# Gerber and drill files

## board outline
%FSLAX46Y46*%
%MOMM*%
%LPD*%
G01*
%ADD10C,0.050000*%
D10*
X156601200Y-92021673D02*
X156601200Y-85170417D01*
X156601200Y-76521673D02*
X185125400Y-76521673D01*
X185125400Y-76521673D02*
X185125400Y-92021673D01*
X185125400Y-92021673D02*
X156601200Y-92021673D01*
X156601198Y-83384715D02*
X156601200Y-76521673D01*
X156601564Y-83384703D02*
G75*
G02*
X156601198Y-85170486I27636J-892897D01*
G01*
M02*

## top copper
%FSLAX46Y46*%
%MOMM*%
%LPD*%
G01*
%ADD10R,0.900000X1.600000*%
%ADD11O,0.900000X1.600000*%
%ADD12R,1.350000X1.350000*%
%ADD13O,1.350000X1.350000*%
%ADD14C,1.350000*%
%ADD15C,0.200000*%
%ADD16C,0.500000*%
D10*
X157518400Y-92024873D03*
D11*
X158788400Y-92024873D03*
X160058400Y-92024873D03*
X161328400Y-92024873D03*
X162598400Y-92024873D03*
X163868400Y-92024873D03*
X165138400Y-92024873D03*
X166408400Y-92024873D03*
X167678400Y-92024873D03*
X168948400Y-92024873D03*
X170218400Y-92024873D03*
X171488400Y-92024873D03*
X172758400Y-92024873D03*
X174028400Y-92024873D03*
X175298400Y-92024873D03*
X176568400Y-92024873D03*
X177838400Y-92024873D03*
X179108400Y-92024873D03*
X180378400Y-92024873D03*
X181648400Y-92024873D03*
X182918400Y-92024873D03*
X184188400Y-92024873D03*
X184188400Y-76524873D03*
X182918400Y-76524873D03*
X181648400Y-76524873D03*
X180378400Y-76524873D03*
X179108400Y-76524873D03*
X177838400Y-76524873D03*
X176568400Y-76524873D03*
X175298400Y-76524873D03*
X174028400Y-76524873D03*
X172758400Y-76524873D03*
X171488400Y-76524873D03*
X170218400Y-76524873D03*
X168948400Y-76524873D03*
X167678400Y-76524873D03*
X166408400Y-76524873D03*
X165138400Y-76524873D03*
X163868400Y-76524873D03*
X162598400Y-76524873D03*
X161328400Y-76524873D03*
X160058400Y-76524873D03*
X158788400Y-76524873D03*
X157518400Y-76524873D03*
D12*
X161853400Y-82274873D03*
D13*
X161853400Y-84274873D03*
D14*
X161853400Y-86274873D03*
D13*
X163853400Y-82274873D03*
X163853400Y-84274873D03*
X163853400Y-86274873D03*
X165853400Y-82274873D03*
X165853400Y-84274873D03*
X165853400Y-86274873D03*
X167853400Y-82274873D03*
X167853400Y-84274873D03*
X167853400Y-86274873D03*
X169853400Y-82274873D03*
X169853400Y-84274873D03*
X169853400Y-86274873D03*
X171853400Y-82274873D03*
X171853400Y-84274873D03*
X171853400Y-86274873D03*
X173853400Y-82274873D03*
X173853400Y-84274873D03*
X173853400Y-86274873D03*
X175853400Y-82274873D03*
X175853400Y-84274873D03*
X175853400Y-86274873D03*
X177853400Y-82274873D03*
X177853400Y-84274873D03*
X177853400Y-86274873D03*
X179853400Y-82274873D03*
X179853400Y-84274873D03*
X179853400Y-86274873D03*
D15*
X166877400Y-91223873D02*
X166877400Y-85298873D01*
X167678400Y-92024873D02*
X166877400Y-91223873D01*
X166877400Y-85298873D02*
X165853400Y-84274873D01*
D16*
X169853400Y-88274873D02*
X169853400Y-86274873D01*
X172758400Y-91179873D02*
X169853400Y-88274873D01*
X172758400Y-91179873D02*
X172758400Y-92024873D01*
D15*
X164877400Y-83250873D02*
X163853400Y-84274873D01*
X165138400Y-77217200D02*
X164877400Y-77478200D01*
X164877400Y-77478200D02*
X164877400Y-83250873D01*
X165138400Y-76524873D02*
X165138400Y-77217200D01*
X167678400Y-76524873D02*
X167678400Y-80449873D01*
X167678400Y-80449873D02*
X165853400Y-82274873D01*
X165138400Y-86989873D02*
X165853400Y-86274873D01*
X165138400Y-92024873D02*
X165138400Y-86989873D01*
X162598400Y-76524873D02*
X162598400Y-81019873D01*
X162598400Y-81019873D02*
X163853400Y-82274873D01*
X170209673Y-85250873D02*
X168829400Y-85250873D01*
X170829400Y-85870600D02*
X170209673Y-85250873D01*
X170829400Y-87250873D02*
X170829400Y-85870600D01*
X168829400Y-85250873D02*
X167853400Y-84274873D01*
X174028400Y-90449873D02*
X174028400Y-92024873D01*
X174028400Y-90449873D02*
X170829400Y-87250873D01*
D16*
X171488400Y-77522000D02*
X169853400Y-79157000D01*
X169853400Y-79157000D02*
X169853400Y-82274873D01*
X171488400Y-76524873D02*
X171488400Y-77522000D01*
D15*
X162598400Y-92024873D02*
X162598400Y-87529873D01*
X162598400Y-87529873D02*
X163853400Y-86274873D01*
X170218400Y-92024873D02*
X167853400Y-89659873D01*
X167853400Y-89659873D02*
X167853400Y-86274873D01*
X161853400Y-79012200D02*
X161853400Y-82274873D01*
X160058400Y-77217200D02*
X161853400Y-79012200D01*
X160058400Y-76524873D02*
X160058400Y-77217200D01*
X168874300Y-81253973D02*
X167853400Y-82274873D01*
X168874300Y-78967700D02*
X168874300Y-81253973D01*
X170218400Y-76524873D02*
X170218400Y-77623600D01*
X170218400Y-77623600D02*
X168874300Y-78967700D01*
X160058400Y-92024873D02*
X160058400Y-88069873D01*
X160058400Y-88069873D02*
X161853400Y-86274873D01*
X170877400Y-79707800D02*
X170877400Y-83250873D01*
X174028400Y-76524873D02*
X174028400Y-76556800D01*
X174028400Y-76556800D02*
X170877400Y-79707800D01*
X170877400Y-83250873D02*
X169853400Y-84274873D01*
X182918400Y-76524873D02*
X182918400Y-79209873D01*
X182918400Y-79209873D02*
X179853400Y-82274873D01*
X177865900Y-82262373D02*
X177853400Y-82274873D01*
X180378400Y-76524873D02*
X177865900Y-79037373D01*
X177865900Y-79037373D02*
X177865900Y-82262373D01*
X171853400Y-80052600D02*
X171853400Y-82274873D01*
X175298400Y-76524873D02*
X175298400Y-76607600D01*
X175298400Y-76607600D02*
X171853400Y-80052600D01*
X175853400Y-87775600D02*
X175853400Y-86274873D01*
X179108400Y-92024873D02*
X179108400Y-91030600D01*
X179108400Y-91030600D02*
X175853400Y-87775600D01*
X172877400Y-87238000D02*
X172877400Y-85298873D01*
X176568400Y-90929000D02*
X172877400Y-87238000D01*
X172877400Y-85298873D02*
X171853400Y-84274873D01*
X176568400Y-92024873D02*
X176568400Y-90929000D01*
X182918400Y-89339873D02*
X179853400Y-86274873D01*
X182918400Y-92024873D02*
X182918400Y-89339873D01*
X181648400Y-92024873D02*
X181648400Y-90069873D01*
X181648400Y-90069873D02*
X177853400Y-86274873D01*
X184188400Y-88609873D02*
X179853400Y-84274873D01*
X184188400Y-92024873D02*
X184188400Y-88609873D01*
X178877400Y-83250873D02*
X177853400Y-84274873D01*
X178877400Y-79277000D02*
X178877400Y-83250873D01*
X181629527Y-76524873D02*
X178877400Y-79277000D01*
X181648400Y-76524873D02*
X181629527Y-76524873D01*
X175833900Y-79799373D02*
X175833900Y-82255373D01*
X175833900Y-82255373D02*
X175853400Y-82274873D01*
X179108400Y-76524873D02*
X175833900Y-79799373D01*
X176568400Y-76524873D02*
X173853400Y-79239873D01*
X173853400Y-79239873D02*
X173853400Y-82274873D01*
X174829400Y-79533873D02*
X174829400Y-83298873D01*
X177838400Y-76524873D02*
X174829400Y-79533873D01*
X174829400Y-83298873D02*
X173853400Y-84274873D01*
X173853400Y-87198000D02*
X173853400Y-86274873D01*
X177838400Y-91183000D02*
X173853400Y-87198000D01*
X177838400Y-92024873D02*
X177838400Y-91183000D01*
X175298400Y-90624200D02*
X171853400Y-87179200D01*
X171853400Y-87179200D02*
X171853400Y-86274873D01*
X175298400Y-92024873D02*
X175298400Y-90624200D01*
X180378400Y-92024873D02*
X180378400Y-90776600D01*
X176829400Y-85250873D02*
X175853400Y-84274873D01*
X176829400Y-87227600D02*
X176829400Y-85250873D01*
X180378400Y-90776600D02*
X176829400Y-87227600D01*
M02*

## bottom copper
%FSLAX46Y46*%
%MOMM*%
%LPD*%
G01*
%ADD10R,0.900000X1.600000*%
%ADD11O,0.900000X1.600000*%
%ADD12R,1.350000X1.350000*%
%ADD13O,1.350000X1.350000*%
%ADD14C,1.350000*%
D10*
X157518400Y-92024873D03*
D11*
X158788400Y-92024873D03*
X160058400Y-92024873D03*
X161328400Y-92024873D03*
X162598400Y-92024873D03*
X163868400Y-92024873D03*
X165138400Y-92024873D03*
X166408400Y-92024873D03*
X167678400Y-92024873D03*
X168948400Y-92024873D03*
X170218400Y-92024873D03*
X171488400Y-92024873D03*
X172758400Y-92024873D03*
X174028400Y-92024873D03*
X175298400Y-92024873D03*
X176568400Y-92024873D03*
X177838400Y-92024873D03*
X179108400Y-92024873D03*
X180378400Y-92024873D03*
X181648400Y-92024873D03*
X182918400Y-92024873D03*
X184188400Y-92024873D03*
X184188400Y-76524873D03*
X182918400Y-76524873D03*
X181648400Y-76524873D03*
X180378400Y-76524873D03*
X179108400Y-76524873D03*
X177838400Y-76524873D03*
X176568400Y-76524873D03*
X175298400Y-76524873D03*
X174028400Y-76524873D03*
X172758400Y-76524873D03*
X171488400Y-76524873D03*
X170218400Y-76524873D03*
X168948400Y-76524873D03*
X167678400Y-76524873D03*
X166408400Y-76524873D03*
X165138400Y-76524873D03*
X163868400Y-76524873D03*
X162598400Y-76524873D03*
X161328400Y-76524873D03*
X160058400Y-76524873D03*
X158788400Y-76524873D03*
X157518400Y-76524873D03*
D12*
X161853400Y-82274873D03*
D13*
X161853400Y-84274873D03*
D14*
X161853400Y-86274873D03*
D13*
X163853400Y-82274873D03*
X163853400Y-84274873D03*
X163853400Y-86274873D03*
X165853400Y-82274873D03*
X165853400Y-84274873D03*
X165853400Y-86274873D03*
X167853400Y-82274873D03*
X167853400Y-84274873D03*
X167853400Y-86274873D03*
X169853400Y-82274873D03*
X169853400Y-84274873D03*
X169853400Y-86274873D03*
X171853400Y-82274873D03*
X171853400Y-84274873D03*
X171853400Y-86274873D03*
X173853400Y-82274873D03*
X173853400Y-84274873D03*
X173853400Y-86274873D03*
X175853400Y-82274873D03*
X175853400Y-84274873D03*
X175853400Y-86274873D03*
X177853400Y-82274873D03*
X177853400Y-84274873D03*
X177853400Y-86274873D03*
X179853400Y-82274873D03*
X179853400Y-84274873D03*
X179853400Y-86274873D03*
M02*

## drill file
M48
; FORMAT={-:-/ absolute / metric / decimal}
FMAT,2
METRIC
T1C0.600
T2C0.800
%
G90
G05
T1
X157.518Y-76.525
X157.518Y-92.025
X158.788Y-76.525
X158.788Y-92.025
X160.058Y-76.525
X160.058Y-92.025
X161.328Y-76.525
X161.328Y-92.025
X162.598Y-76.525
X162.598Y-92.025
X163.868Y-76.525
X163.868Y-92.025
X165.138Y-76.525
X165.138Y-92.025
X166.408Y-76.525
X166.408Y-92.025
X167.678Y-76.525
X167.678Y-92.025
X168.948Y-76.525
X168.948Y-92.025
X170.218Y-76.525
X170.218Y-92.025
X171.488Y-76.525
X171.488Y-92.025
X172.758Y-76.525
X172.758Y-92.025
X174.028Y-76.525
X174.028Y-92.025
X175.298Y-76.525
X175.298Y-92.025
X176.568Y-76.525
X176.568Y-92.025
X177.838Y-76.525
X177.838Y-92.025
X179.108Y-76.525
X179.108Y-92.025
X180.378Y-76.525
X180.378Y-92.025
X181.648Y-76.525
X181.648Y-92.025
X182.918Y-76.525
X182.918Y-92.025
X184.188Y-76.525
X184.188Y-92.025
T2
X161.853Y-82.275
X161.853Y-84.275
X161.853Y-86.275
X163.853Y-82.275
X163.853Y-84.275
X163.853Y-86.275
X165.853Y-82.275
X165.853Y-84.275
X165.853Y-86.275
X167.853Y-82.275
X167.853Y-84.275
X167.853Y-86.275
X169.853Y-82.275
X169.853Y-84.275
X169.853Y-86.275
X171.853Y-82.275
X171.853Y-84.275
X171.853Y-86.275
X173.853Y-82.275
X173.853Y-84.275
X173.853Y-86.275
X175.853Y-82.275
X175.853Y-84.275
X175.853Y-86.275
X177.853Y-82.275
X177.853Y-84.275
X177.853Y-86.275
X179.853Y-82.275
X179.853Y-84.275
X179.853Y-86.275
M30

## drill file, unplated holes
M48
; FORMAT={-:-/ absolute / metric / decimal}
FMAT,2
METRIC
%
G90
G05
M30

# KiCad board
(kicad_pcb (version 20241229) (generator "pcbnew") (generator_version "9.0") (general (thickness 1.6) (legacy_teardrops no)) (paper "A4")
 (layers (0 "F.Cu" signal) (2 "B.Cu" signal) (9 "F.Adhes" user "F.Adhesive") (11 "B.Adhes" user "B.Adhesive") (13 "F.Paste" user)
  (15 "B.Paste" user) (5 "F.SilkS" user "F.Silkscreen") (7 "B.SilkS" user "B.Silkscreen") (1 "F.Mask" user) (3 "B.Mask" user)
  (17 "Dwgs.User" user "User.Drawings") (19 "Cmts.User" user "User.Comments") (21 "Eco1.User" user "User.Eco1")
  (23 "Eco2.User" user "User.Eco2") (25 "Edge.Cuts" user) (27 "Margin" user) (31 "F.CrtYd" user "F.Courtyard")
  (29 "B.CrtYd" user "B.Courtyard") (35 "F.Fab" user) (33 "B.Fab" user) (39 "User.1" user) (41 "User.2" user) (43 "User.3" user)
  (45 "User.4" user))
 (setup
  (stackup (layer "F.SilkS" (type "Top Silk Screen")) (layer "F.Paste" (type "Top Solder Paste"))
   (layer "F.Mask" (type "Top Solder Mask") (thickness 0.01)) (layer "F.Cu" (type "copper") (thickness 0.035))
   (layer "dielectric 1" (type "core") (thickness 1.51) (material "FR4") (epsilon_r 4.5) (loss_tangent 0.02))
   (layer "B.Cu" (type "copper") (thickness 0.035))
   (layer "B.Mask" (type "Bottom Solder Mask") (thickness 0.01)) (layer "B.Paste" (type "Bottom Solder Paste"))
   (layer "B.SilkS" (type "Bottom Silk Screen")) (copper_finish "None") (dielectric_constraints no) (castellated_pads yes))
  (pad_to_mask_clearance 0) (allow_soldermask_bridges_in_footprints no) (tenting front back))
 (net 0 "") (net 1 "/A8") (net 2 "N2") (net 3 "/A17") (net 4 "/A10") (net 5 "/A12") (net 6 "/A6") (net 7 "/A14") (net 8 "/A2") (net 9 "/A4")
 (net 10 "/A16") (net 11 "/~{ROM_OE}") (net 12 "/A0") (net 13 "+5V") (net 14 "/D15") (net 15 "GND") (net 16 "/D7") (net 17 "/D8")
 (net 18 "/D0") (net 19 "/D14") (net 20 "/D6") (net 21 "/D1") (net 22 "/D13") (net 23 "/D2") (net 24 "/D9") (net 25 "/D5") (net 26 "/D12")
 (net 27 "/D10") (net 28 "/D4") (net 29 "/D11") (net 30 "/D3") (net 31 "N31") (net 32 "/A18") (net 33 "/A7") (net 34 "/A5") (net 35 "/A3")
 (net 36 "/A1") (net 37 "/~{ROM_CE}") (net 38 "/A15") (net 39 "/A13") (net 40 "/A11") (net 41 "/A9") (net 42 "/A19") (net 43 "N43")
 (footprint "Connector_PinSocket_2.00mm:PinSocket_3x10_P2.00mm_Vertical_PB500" (layer "F.Cu") (at 161.8534 82.274873 90)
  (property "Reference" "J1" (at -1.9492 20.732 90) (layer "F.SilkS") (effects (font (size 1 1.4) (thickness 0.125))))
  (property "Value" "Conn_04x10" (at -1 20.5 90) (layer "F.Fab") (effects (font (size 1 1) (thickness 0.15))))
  (pad "1" thru_hole rect (at 0 0 90) (size 1.35 1.35) (drill 0.8) (layers "*.Cu" "*.Mask") (remove_unused_layers no) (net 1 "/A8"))
  (pad "2" thru_hole oval (at -2 0 90) (size 1.35 1.35) (drill 0.8) (layers "*.Cu" "*.Mask") (remove_unused_layers no) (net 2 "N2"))
  (pad "3" thru_hole circle (at -4 0 90) (size 1.35 1.35) (drill 0.8) (layers "*.Cu" "*.Mask") (remove_unused_layers no) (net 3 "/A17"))
  (pad "4" thru_hole oval (at 0 2 90) (size 1.35 1.35) (drill 0.8) (layers "*.Cu" "*.Mask") (remove_unused_layers no) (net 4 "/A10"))
  (pad "5" thru_hole oval (at -2 2 90) (size 1.35 1.35) (drill 0.8) (layers "*.Cu" "*.Mask") (remove_unused_layers no) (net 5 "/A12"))
  (pad "6" thru_hole oval (at -4 2 90) (size 1.35 1.35) (drill 0.8) (layers "*.Cu" "*.Mask") (remove_unused_layers no) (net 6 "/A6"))
  (pad "7" thru_hole oval (at 0 4 90) (size 1.35 1.35) (drill 0.8) (layers "*.Cu" "*.Mask") (remove_unused_layers no) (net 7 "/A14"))
  (pad "8" thru_hole oval (at -2 4 90) (size 1.35 1.35) (drill 0.8) (layers "*.Cu" "*.Mask") (remove_unused_layers no) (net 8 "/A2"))
  (pad "9" thru_hole oval (at -4 4 90) (size 1.35 1.35) (drill 0.8) (layers "*.Cu" "*.Mask") (remove_unused_layers no) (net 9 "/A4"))
  (pad "10" thru_hole oval (at 0 6 90) (size 1.35 1.35) (drill 0.8) (layers "*.Cu" "*.Mask") (remove_unused_layers no) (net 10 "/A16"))
  (pad "11" thru_hole oval (at -2 6 90) (size 1.35 1.35) (drill 0.8) (layers "*.Cu" "*.Mask") (remove_unused_layers no)
   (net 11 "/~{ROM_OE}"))
  (pad "12" thru_hole oval (at -4 6 90) (size 1.35 1.35) (drill 0.8) (layers "*.Cu" "*.Mask") (remove_unused_layers no) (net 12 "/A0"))
  (pad "13" thru_hole oval (at 0 8 90) (size 1.35 1.35) (drill 0.8) (layers "*.Cu" "*.Mask") (remove_unused_layers no) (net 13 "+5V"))
  (pad "14" thru_hole oval (at -2 8 90) (size 1.35 1.35) (drill 0.8) (layers "*.Cu" "*.Mask") (remove_unused_layers no) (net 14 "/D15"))
  (pad "15" thru_hole oval (at -4 8 90) (size 1.35 1.35) (drill 0.8) (layers "*.Cu" "*.Mask") (remove_unused_layers no) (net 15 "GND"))
  (pad "16" thru_hole oval (at 0 10 90) (size 1.35 1.35) (drill 0.8) (layers "*.Cu" "*.Mask") (remove_unused_layers no) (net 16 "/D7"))
  (pad "17" thru_hole oval (at -2 10 90) (size 1.35 1.35) (drill 0.8) (layers "*.Cu" "*.Mask") (remove_unused_layers no) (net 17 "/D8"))
  (pad "18" thru_hole oval (at -4 10 90) (size 1.35 1.35) (drill 0.8) (layers "*.Cu" "*.Mask") (remove_unused_layers no) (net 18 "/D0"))
  (pad "19" thru_hole oval (at 0 12 90) (size 1.35 1.35) (drill 0.8) (layers "*.Cu" "*.Mask") (remove_unused_layers no) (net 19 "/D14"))
  (pad "20" thru_hole oval (at -2 12 90) (size 1.35 1.35) (drill 0.8) (layers "*.Cu" "*.Mask") (remove_unused_layers no) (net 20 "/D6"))
  (pad "21" thru_hole oval (at -4 12 90) (size 1.35 1.35) (drill 0.8) (layers "*.Cu" "*.Mask") (remove_unused_layers no) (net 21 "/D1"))
  (pad "22" thru_hole oval (at 0 14 90) (size 1.35 1.35) (drill 0.8) (layers "*.Cu" "*.Mask") (remove_unused_layers no) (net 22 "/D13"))
  (pad "23" thru_hole oval (at -2 14 90) (size 1.35 1.35) (drill 0.8) (layers "*.Cu" "*.Mask") (remove_unused_layers no) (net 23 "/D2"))
  (pad "24" thru_hole oval (at -4 14 90) (size 1.35 1.35) (drill 0.8) (layers "*.Cu" "*.Mask") (remove_unused_layers no) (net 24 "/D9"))
  (pad "25" thru_hole oval (at 0 16 90) (size 1.35 1.35) (drill 0.8) (layers "*.Cu" "*.Mask") (remove_unused_layers no) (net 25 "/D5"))
  (pad "26" thru_hole oval (at -2 16 90) (size 1.35 1.35) (drill 0.8) (layers "*.Cu" "*.Mask") (remove_unused_layers no) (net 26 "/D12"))
  (pad "27" thru_hole oval (at -4 16 90) (size 1.35 1.35) (drill 0.8) (layers "*.Cu" "*.Mask") (remove_unused_layers no) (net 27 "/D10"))
  (pad "28" thru_hole oval (at 0 18 90) (size 1.35 1.35) (drill 0.8) (layers "*.Cu" "*.Mask") (remove_unused_layers no) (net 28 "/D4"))
  (pad "29" thru_hole oval (at -2 18 90) (size 1.35 1.35) (drill 0.8) (layers "*.Cu" "*.Mask") (remove_unused_layers no) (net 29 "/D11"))
  (pad "30" thru_hole oval (at -4 18 90) (size 1.35 1.35) (drill 0.8) (layers "*.Cu" "*.Mask") (remove_unused_layers no) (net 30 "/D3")))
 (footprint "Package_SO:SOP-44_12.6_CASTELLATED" (layer "F.Cu") (at 170.8534 84.274873 90)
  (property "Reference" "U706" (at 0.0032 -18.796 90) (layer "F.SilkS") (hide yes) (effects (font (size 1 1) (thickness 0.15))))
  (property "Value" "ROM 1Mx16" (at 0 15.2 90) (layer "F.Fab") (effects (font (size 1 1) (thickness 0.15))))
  (pad "1" thru_hole rect (at -7.75 -13.335 90) (size 1.6 0.9) (drill 0.6) (layers "*.Cu" "*.Mask") (remove_unused_layers no) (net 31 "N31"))
  (pad "2" thru_hole oval (at -7.75 -12.065 90) (size 1.6 0.9) (drill 0.6) (layers "*.Cu" "*.Mask") (remove_unused_layers no)
   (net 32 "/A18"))
  (pad "3" thru_hole oval (at -7.75 -10.795 90) (size 1.6 0.9) (drill 0.6) (layers "*.Cu" "*.Mask") (remove_unused_layers no) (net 3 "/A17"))
  (pad "4" thru_hole oval (at -7.75 -9.525 90) (size 1.6 0.9) (drill 0.6) (layers "*.Cu" "*.Mask") (remove_unused_layers no) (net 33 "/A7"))
  (pad "5" thru_hole oval (at -7.75 -8.255 90) (size 1.6 0.9) (drill 0.6) (layers "*.Cu" "*.Mask") (remove_unused_layers no) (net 6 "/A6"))
  (pad "6" thru_hole oval (at -7.75 -6.985 90) (size 1.6 0.9) (drill 0.6) (layers "*.Cu" "*.Mask") (remove_unused_layers no) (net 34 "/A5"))
  (pad "7" thru_hole oval (at -7.75 -5.715 90) (size 1.6 0.9) (drill 0.6) (layers "*.Cu" "*.Mask") (remove_unused_layers no) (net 9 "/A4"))
  (pad "8" thru_hole oval (at -7.75 -4.445 90) (size 1.6 0.9) (drill 0.6) (layers "*.Cu" "*.Mask") (remove_unused_layers no) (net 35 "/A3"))
  (pad "9" thru_hole oval (at -7.75 -3.175 90) (size 1.6 0.9) (drill 0.6) (layers "*.Cu" "*.Mask") (remove_unused_layers no) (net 8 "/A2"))
  (pad "10" thru_hole oval (at -7.75 -1.905 90) (size 1.6 0.9) (drill 0.6) (layers "*.Cu" "*.Mask") (remove_unused_layers no) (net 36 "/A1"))
  (pad "11" thru_hole oval (at -7.75 -0.635 90) (size 1.6 0.9) (drill 0.6) (layers "*.Cu" "*.Mask") (remove_unused_layers no) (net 12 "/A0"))
  (pad "12" thru_hole oval (at -7.75 0.635 90) (size 1.6 0.9) (drill 0.6) (layers "*.Cu" "*.Mask") (remove_unused_layers no)
   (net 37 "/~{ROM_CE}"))
  (pad "13" thru_hole oval (at -7.75 1.905 90) (size 1.6 0.9) (drill 0.6) (layers "*.Cu" "*.Mask") (remove_unused_layers no) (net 15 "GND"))
  (pad "14" thru_hole oval (at -7.75 3.175 90) (size 1.6 0.9) (drill 0.6) (layers "*.Cu" "*.Mask") (remove_unused_layers no)
   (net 11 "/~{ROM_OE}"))
  (pad "15" thru_hole oval (at -7.75 4.445 90) (size 1.6 0.9) (drill 0.6) (layers "*.Cu" "*.Mask") (remove_unused_layers no) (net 18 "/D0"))
  (pad "16" thru_hole oval (at -7.75 5.715 90) (size 1.6 0.9) (drill 0.6) (layers "*.Cu" "*.Mask") (remove_unused_layers no) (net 17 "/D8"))
  (pad "17" thru_hole oval (at -7.75 6.985 90) (size 1.6 0.9) (drill 0.6) (layers "*.Cu" "*.Mask") (remove_unused_layers no) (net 21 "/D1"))
  (pad "18" thru_hole oval (at -7.75 8.255 90) (size 1.6 0.9) (drill 0.6) (layers "*.Cu" "*.Mask") (remove_unused_layers no) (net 24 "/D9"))
  (pad "19" thru_hole oval (at -7.75 9.525 90) (size 1.6 0.9) (drill 0.6) (layers "*.Cu" "*.Mask") (remove_unused_layers no) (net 23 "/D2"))
  (pad "20" thru_hole oval (at -7.75 10.795 90) (size 1.6 0.9) (drill 0.6) (layers "*.Cu" "*.Mask") (remove_unused_layers no)
   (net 27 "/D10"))
  (pad "21" thru_hole oval (at -7.75 12.065 90) (size 1.6 0.9) (drill 0.6) (layers "*.Cu" "*.Mask") (remove_unused_layers no) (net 30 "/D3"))
  (pad "22" thru_hole oval (at -7.75 13.335 90) (size 1.6 0.9) (drill 0.6) (layers "*.Cu" "*.Mask") (remove_unused_layers no)
   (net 29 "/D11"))
  (pad "23" thru_hole oval (at 7.75 13.335 90) (size 1.6 0.9) (drill 0.6) (layers "*.Cu" "*.Mask") (remove_unused_layers no) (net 13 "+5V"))
  (pad "24" thru_hole oval (at 7.75 12.065 90) (size 1.6 0.9) (drill 0.6) (layers "*.Cu" "*.Mask") (remove_unused_layers no) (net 28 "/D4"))
  (pad "25" thru_hole oval (at 7.75 10.795 90) (size 1.6 0.9) (drill 0.6) (layers "*.Cu" "*.Mask") (remove_unused_layers no) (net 26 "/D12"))
  (pad "26" thru_hole oval (at 7.75 9.525 90) (size 1.6 0.9) (drill 0.6) (layers "*.Cu" "*.Mask") (remove_unused_layers no) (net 25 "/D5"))
  (pad "27" thru_hole oval (at 7.75 8.255 90) (size 1.6 0.9) (drill 0.6) (layers "*.Cu" "*.Mask") (remove_unused_layers no) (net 22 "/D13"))
  (pad "28" thru_hole oval (at 7.75 6.985 90) (size 1.6 0.9) (drill 0.6) (layers "*.Cu" "*.Mask") (remove_unused_layers no) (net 20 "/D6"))
  (pad "29" thru_hole oval (at 7.75 5.715 90) (size 1.6 0.9) (drill 0.6) (layers "*.Cu" "*.Mask") (remove_unused_layers no) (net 19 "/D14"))
  (pad "30" thru_hole oval (at 7.75 4.445 90) (size 1.6 0.9) (drill 0.6) (layers "*.Cu" "*.Mask") (remove_unused_layers no) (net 16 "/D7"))
  (pad "31" thru_hole oval (at 7.75 3.175 90) (size 1.6 0.9) (drill 0.6) (layers "*.Cu" "*.Mask") (remove_unused_layers no) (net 14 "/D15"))
  (pad "32" thru_hole oval (at 7.75 1.905 90) (size 1.6 0.9) (drill 0.6) (layers "*.Cu" "*.Mask") (remove_unused_layers no) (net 15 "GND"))
  (pad "33" thru_hole oval (at 7.75 0.635 90) (size 1.6 0.9) (drill 0.6) (layers "*.Cu" "*.Mask") (remove_unused_layers no) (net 13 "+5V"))
  (pad "34" thru_hole oval (at 7.75 -0.635 90) (size 1.6 0.9) (drill 0.6) (layers "*.Cu" "*.Mask") (remove_unused_layers no) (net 10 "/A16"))
  (pad "35" thru_hole oval (at 7.75 -1.905 90) (size 1.6 0.9) (drill 0.6) (layers "*.Cu" "*.Mask") (remove_unused_layers no) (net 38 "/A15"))
  (pad "36" thru_hole oval (at 7.75 -3.175 90) (size 1.6 0.9) (drill 0.6) (layers "*.Cu" "*.Mask") (remove_unused_layers no) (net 7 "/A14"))
  (pad "37" thru_hole oval (at 7.75 -4.445 90) (size 1.6 0.9) (drill 0.6) (layers "*.Cu" "*.Mask") (remove_unused_layers no) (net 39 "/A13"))
  (pad "38" thru_hole oval (at 7.75 -5.715 90) (size 1.6 0.9) (drill 0.6) (layers "*.Cu" "*.Mask") (remove_unused_layers no) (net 5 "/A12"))
  (pad "39" thru_hole oval (at 7.75 -6.985 90) (size 1.6 0.9) (drill 0.6) (layers "*.Cu" "*.Mask") (remove_unused_layers no) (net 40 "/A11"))
  (pad "40" thru_hole oval (at 7.75 -8.255 90) (size 1.6 0.9) (drill 0.6) (layers "*.Cu" "*.Mask") (remove_unused_layers no) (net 4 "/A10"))
  (pad "41" thru_hole oval (at 7.75 -9.525 90) (size 1.6 0.9) (drill 0.6) (layers "*.Cu" "*.Mask") (remove_unused_layers no) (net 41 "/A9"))
  (pad "42" thru_hole oval (at 7.75 -10.795 90) (size 1.6 0.9) (drill 0.6) (layers "*.Cu" "*.Mask") (remove_unused_layers no) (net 1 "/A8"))
  (pad "43" thru_hole oval (at 7.75 -12.065 90) (size 1.6 0.9) (drill 0.6) (layers "*.Cu" "*.Mask") (remove_unused_layers no)
   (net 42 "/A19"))
  (pad "44" thru_hole oval (at 7.75 -13.335 90) (size 1.6 0.9) (drill 0.6) (layers "*.Cu" "*.Mask") (remove_unused_layers no) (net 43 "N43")))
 (gr_line (start 156.6012 92.021673) (end 156.6012 85.170417) (stroke (width 0.05) (type default)) (layer "Edge.Cuts"))
 (gr_line (start 156.6012 76.521673) (end 185.1254 76.521673) (stroke (width 0.05) (type default)) (layer "Edge.Cuts"))
 (gr_line (start 185.1254 76.521673) (end 185.1254 92.021673) (stroke (width 0.05) (type default)) (layer "Edge.Cuts"))
 (gr_line (start 185.1254 92.021673) (end 156.6012 92.021673) (stroke (width 0.05) (type default)) (layer "Edge.Cuts"))
 (gr_line (start 156.601198 83.384715) (end 156.6012 76.521673) (stroke (width 0.05) (type default)) (layer "Edge.Cuts"))
 (gr_arc (start 156.601564 83.384703) (mid 157.522444 84.277748) (end 156.6012 85.170417) (stroke (width 0.05) (type default))
  (layer "Edge.Cuts"))
 (segment (start 166.8774 91.223873) (end 166.8774 85.298873) (width 0.2) (layer "F.Cu") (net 8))
 (segment (start 167.6784 92.024873) (end 166.8774 91.223873) (width 0.2) (layer "F.Cu") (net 8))
 (segment (start 166.8774 85.298873) (end 165.8534 84.274873) (width 0.2) (layer "F.Cu") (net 8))
 (segment (start 169.8534 88.274873) (end 169.8534 86.274873) (width 0.5) (layer "F.Cu") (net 15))
 (segment (start 172.7584 91.179873) (end 169.8534 88.274873) (width 0.5) (layer "F.Cu") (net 15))
 (segment (start 172.7584 91.179873) (end 172.7584 92.024873) (width 0.5) (layer "F.Cu") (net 15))
 (segment (start 164.8774 83.250873) (end 163.8534 84.274873) (width 0.2) (layer "F.Cu") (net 5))
 (segment (start 165.1384 77.2172) (end 164.8774 77.4782) (width 0.2) (layer "F.Cu") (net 5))
 (segment (start 164.8774 77.4782) (end 164.8774 83.250873) (width 0.2) (layer "F.Cu") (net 5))
 (segment (start 165.1384 76.524873) (end 165.1384 77.2172) (width 0.2) (layer "F.Cu") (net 5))
 (segment (start 167.6784 76.524873) (end 167.6784 80.449873) (width 0.2) (layer "F.Cu") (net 7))
 (segment (start 167.6784 80.449873) (end 165.8534 82.274873) (width 0.2) (layer "F.Cu") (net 7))
 (segment (start 165.1384 86.989873) (end 165.8534 86.274873) (width 0.2) (layer "F.Cu") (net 9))
 (segment (start 165.1384 92.024873) (end 165.1384 86.989873) (width 0.2) (layer "F.Cu") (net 9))
 (segment (start 162.5984 76.524873) (end 162.5984 81.019873) (width 0.2) (layer "F.Cu") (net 4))
 (segment (start 162.5984 81.019873) (end 163.8534 82.274873) (width 0.2) (layer "F.Cu") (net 4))
 (segment (start 170.209673 85.250873) (end 168.8294 85.250873) (width 0.2) (layer "F.Cu") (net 11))
 (segment (start 170.8294 85.8706) (end 170.209673 85.250873) (width 0.2) (layer "F.Cu") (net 11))
 (segment (start 170.8294 87.250873) (end 170.8294 85.8706) (width 0.2) (layer "F.Cu") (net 11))
 (segment (start 168.8294 85.250873) (end 167.8534 84.274873) (width 0.2) (layer "F.Cu") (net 11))
 (segment (start 174.0284 90.449873) (end 174.0284 92.024873) (width 0.2) (layer "F.Cu") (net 11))
 (segment (start 174.0284 90.449873) (end 170.8294 87.250873) (width 0.2) (layer "F.Cu") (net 11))
 (segment (start 171.4884 77.522) (end 169.8534 79.157) (width 0.5) (layer "F.Cu") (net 13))
 (segment (start 169.8534 79.157) (end 169.8534 82.274873) (width 0.5) (layer "F.Cu") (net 13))
 (segment (start 171.4884 76.524873) (end 171.4884 77.522) (width 0.5) (layer "F.Cu") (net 13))
 (segment (start 162.5984 92.024873) (end 162.5984 87.529873) (width 0.2) (layer "F.Cu") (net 6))
 (segment (start 162.5984 87.529873) (end 163.8534 86.274873) (width 0.2) (layer "F.Cu") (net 6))
 (segment (start 170.2184 92.024873) (end 167.8534 89.659873) (width 0.2) (layer "F.Cu") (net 12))
 (segment (start 167.8534 89.659873) (end 167.8534 86.274873) (width 0.2) (layer "F.Cu") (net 12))
 (segment (start 161.8534 79.0122) (end 161.8534 82.274873) (width 0.2) (layer "F.Cu") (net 1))
 (segment (start 160.0584 77.2172) (end 161.8534 79.0122) (width 0.2) (layer "F.Cu") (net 1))
 (segment (start 160.0584 76.524873) (end 160.0584 77.2172) (width 0.2) (layer "F.Cu") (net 1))
 (segment (start 168.8743 81.253973) (end 167.8534 82.274873) (width 0.2) (layer "F.Cu") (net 10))
 (segment (start 168.8743 78.9677) (end 168.8743 81.253973) (width 0.2) (layer "F.Cu") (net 10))
 (segment (start 170.2184 76.524873) (end 170.2184 77.6236) (width 0.2) (layer "F.Cu") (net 10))
 (segment (start 170.2184 77.6236) (end 168.8743 78.9677) (width 0.2) (layer "F.Cu") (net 10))
 (segment (start 160.0584 92.024873) (end 160.0584 88.069873) (width 0.2) (layer "F.Cu") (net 3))
 (segment (start 160.0584 88.069873) (end 161.8534 86.274873) (width 0.2) (layer "F.Cu") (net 3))
 (segment (start 170.8774 79.7078) (end 170.8774 83.250873) (width 0.2) (layer "F.Cu") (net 14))
 (segment (start 174.0284 76.524873) (end 174.0284 76.5568) (width 0.2) (layer "F.Cu") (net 14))
 (segment (start 174.0284 76.5568) (end 170.8774 79.7078) (width 0.2) (layer "F.Cu") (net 14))
 (segment (start 170.8774 83.250873) (end 169.8534 84.274873) (width 0.2) (layer "F.Cu") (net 14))
 (segment (start 182.9184 76.524873) (end 182.9184 79.209873) (width 0.2) (layer "F.Cu") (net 28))
 (segment (start 182.9184 79.209873) (end 179.8534 82.274873) (width 0.2) (layer "F.Cu") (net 28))
 (segment (start 177.8659 82.262373) (end 177.8534 82.274873) (width 0.2) (layer "F.Cu") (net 25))
 (segment (start 180.3784 76.524873) (end 177.8659 79.037373) (width 0.2) (layer "F.Cu") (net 25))
 (segment (start 177.8659 79.037373) (end 177.8659 82.262373) (width 0.2) (layer "F.Cu") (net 25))
 (segment (start 171.8534 80.0526) (end 171.8534 82.274873) (width 0.2) (layer "F.Cu") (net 16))
 (segment (start 175.2984 76.524873) (end 175.2984 76.6076) (width 0.2) (layer "F.Cu") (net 16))
 (segment (start 175.2984 76.6076) (end 171.8534 80.0526) (width 0.2) (layer "F.Cu") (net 16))
 (segment (start 175.8534 87.7756) (end 175.8534 86.274873) (width 0.2) (layer "F.Cu") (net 24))
 (segment (start 179.1084 92.024873) (end 179.1084 91.0306) (width 0.2) (layer "F.Cu") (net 24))
 (segment (start 179.1084 91.0306) (end 175.8534 87.7756) (width 0.2) (layer "F.Cu") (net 24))
 (segment (start 172.8774 87.238) (end 172.8774 85.298873) (width 0.2) (layer "F.Cu") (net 17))
 (segment (start 176.5684 90.929) (end 172.8774 87.238) (width 0.2) (layer "F.Cu") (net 17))
 (segment (start 172.8774 85.298873) (end 171.8534 84.274873) (width 0.2) (layer "F.Cu") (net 17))
 (segment (start 176.5684 92.024873) (end 176.5684 90.929) (width 0.2) (layer "F.Cu") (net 17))
 (segment (start 182.9184 89.339873) (end 179.8534 86.274873) (width 0.2) (layer "F.Cu") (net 30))
 (segment (start 182.9184 92.024873) (end 182.9184 89.339873) (width 0.2) (layer "F.Cu") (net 30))
 (segment (start 181.6484 92.024873) (end 181.6484 90.069873) (width 0.2) (layer "F.Cu") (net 27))
 (segment (start 181.6484 90.069873) (end 177.8534 86.274873) (width 0.2) (layer "F.Cu") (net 27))
 (segment (start 184.1884 88.609873) (end 179.8534 84.274873) (width 0.2) (layer "F.Cu") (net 29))
 (segment (start 184.1884 92.024873) (end 184.1884 88.609873) (width 0.2) (layer "F.Cu") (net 29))
 (segment (start 178.8774 83.250873) (end 177.8534 84.274873) (width 0.2) (layer "F.Cu") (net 26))
 (segment (start 178.8774 79.277) (end 178.8774 83.250873) (width 0.2) (layer "F.Cu") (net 26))
 (segment (start 181.629527 76.524873) (end 178.8774 79.277) (width 0.2) (layer "F.Cu") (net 26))
 (segment (start 181.6484 76.524873) (end 181.629527 76.524873) (width 0.2) (layer "F.Cu") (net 26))
 (segment (start 175.8339 79.799373) (end 175.8339 82.255373) (width 0.2) (layer "F.Cu") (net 22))
 (segment (start 175.8339 82.255373) (end 175.8534 82.274873) (width 0.2) (layer "F.Cu") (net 22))
 (segment (start 179.1084 76.524873) (end 175.8339 79.799373) (width 0.2) (layer "F.Cu") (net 22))
 (segment (start 176.5684 76.524873) (end 173.8534 79.239873) (width 0.2) (layer "F.Cu") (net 19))
 (segment (start 173.8534 79.239873) (end 173.8534 82.274873) (width 0.2) (layer "F.Cu") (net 19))
 (segment (start 174.8294 79.533873) (end 174.8294 83.298873) (width 0.2) (layer "F.Cu") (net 20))
 (segment (start 177.8384 76.524873) (end 174.8294 79.533873) (width 0.2) (layer "F.Cu") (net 20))
 (segment (start 174.8294 83.298873) (end 173.8534 84.274873) (width 0.2) (layer "F.Cu") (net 20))
 (segment (start 173.8534 87.198) (end 173.8534 86.274873) (width 0.2) (layer "F.Cu") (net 21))
 (segment (start 177.8384 91.183) (end 173.8534 87.198) (width 0.2) (layer "F.Cu") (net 21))
 (segment (start 177.8384 92.024873) (end 177.8384 91.183) (width 0.2) (layer "F.Cu") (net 21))
 (segment (start 175.2984 90.6242) (end 171.8534 87.1792) (width 0.2) (layer "F.Cu") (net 18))
 (segment (start 171.8534 87.1792) (end 171.8534 86.274873) (width 0.2) (layer "F.Cu") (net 18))
 (segment (start 175.2984 92.024873) (end 175.2984 90.6242) (width 0.2) (layer "F.Cu") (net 18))
 (segment (start 180.3784 92.024873) (end 180.3784 90.7766) (width 0.2) (layer "F.Cu") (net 23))
 (segment (start 176.8294 85.250873) (end 175.8534 84.274873) (width 0.2) (layer "F.Cu") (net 23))
 (segment (start 176.8294 87.2276) (end 176.8294 85.250873) (width 0.2) (layer "F.Cu") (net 23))
 (segment (start 180.3784 90.7766) (end 176.8294 87.2276) (width 0.2) (layer "F.Cu") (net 23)))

